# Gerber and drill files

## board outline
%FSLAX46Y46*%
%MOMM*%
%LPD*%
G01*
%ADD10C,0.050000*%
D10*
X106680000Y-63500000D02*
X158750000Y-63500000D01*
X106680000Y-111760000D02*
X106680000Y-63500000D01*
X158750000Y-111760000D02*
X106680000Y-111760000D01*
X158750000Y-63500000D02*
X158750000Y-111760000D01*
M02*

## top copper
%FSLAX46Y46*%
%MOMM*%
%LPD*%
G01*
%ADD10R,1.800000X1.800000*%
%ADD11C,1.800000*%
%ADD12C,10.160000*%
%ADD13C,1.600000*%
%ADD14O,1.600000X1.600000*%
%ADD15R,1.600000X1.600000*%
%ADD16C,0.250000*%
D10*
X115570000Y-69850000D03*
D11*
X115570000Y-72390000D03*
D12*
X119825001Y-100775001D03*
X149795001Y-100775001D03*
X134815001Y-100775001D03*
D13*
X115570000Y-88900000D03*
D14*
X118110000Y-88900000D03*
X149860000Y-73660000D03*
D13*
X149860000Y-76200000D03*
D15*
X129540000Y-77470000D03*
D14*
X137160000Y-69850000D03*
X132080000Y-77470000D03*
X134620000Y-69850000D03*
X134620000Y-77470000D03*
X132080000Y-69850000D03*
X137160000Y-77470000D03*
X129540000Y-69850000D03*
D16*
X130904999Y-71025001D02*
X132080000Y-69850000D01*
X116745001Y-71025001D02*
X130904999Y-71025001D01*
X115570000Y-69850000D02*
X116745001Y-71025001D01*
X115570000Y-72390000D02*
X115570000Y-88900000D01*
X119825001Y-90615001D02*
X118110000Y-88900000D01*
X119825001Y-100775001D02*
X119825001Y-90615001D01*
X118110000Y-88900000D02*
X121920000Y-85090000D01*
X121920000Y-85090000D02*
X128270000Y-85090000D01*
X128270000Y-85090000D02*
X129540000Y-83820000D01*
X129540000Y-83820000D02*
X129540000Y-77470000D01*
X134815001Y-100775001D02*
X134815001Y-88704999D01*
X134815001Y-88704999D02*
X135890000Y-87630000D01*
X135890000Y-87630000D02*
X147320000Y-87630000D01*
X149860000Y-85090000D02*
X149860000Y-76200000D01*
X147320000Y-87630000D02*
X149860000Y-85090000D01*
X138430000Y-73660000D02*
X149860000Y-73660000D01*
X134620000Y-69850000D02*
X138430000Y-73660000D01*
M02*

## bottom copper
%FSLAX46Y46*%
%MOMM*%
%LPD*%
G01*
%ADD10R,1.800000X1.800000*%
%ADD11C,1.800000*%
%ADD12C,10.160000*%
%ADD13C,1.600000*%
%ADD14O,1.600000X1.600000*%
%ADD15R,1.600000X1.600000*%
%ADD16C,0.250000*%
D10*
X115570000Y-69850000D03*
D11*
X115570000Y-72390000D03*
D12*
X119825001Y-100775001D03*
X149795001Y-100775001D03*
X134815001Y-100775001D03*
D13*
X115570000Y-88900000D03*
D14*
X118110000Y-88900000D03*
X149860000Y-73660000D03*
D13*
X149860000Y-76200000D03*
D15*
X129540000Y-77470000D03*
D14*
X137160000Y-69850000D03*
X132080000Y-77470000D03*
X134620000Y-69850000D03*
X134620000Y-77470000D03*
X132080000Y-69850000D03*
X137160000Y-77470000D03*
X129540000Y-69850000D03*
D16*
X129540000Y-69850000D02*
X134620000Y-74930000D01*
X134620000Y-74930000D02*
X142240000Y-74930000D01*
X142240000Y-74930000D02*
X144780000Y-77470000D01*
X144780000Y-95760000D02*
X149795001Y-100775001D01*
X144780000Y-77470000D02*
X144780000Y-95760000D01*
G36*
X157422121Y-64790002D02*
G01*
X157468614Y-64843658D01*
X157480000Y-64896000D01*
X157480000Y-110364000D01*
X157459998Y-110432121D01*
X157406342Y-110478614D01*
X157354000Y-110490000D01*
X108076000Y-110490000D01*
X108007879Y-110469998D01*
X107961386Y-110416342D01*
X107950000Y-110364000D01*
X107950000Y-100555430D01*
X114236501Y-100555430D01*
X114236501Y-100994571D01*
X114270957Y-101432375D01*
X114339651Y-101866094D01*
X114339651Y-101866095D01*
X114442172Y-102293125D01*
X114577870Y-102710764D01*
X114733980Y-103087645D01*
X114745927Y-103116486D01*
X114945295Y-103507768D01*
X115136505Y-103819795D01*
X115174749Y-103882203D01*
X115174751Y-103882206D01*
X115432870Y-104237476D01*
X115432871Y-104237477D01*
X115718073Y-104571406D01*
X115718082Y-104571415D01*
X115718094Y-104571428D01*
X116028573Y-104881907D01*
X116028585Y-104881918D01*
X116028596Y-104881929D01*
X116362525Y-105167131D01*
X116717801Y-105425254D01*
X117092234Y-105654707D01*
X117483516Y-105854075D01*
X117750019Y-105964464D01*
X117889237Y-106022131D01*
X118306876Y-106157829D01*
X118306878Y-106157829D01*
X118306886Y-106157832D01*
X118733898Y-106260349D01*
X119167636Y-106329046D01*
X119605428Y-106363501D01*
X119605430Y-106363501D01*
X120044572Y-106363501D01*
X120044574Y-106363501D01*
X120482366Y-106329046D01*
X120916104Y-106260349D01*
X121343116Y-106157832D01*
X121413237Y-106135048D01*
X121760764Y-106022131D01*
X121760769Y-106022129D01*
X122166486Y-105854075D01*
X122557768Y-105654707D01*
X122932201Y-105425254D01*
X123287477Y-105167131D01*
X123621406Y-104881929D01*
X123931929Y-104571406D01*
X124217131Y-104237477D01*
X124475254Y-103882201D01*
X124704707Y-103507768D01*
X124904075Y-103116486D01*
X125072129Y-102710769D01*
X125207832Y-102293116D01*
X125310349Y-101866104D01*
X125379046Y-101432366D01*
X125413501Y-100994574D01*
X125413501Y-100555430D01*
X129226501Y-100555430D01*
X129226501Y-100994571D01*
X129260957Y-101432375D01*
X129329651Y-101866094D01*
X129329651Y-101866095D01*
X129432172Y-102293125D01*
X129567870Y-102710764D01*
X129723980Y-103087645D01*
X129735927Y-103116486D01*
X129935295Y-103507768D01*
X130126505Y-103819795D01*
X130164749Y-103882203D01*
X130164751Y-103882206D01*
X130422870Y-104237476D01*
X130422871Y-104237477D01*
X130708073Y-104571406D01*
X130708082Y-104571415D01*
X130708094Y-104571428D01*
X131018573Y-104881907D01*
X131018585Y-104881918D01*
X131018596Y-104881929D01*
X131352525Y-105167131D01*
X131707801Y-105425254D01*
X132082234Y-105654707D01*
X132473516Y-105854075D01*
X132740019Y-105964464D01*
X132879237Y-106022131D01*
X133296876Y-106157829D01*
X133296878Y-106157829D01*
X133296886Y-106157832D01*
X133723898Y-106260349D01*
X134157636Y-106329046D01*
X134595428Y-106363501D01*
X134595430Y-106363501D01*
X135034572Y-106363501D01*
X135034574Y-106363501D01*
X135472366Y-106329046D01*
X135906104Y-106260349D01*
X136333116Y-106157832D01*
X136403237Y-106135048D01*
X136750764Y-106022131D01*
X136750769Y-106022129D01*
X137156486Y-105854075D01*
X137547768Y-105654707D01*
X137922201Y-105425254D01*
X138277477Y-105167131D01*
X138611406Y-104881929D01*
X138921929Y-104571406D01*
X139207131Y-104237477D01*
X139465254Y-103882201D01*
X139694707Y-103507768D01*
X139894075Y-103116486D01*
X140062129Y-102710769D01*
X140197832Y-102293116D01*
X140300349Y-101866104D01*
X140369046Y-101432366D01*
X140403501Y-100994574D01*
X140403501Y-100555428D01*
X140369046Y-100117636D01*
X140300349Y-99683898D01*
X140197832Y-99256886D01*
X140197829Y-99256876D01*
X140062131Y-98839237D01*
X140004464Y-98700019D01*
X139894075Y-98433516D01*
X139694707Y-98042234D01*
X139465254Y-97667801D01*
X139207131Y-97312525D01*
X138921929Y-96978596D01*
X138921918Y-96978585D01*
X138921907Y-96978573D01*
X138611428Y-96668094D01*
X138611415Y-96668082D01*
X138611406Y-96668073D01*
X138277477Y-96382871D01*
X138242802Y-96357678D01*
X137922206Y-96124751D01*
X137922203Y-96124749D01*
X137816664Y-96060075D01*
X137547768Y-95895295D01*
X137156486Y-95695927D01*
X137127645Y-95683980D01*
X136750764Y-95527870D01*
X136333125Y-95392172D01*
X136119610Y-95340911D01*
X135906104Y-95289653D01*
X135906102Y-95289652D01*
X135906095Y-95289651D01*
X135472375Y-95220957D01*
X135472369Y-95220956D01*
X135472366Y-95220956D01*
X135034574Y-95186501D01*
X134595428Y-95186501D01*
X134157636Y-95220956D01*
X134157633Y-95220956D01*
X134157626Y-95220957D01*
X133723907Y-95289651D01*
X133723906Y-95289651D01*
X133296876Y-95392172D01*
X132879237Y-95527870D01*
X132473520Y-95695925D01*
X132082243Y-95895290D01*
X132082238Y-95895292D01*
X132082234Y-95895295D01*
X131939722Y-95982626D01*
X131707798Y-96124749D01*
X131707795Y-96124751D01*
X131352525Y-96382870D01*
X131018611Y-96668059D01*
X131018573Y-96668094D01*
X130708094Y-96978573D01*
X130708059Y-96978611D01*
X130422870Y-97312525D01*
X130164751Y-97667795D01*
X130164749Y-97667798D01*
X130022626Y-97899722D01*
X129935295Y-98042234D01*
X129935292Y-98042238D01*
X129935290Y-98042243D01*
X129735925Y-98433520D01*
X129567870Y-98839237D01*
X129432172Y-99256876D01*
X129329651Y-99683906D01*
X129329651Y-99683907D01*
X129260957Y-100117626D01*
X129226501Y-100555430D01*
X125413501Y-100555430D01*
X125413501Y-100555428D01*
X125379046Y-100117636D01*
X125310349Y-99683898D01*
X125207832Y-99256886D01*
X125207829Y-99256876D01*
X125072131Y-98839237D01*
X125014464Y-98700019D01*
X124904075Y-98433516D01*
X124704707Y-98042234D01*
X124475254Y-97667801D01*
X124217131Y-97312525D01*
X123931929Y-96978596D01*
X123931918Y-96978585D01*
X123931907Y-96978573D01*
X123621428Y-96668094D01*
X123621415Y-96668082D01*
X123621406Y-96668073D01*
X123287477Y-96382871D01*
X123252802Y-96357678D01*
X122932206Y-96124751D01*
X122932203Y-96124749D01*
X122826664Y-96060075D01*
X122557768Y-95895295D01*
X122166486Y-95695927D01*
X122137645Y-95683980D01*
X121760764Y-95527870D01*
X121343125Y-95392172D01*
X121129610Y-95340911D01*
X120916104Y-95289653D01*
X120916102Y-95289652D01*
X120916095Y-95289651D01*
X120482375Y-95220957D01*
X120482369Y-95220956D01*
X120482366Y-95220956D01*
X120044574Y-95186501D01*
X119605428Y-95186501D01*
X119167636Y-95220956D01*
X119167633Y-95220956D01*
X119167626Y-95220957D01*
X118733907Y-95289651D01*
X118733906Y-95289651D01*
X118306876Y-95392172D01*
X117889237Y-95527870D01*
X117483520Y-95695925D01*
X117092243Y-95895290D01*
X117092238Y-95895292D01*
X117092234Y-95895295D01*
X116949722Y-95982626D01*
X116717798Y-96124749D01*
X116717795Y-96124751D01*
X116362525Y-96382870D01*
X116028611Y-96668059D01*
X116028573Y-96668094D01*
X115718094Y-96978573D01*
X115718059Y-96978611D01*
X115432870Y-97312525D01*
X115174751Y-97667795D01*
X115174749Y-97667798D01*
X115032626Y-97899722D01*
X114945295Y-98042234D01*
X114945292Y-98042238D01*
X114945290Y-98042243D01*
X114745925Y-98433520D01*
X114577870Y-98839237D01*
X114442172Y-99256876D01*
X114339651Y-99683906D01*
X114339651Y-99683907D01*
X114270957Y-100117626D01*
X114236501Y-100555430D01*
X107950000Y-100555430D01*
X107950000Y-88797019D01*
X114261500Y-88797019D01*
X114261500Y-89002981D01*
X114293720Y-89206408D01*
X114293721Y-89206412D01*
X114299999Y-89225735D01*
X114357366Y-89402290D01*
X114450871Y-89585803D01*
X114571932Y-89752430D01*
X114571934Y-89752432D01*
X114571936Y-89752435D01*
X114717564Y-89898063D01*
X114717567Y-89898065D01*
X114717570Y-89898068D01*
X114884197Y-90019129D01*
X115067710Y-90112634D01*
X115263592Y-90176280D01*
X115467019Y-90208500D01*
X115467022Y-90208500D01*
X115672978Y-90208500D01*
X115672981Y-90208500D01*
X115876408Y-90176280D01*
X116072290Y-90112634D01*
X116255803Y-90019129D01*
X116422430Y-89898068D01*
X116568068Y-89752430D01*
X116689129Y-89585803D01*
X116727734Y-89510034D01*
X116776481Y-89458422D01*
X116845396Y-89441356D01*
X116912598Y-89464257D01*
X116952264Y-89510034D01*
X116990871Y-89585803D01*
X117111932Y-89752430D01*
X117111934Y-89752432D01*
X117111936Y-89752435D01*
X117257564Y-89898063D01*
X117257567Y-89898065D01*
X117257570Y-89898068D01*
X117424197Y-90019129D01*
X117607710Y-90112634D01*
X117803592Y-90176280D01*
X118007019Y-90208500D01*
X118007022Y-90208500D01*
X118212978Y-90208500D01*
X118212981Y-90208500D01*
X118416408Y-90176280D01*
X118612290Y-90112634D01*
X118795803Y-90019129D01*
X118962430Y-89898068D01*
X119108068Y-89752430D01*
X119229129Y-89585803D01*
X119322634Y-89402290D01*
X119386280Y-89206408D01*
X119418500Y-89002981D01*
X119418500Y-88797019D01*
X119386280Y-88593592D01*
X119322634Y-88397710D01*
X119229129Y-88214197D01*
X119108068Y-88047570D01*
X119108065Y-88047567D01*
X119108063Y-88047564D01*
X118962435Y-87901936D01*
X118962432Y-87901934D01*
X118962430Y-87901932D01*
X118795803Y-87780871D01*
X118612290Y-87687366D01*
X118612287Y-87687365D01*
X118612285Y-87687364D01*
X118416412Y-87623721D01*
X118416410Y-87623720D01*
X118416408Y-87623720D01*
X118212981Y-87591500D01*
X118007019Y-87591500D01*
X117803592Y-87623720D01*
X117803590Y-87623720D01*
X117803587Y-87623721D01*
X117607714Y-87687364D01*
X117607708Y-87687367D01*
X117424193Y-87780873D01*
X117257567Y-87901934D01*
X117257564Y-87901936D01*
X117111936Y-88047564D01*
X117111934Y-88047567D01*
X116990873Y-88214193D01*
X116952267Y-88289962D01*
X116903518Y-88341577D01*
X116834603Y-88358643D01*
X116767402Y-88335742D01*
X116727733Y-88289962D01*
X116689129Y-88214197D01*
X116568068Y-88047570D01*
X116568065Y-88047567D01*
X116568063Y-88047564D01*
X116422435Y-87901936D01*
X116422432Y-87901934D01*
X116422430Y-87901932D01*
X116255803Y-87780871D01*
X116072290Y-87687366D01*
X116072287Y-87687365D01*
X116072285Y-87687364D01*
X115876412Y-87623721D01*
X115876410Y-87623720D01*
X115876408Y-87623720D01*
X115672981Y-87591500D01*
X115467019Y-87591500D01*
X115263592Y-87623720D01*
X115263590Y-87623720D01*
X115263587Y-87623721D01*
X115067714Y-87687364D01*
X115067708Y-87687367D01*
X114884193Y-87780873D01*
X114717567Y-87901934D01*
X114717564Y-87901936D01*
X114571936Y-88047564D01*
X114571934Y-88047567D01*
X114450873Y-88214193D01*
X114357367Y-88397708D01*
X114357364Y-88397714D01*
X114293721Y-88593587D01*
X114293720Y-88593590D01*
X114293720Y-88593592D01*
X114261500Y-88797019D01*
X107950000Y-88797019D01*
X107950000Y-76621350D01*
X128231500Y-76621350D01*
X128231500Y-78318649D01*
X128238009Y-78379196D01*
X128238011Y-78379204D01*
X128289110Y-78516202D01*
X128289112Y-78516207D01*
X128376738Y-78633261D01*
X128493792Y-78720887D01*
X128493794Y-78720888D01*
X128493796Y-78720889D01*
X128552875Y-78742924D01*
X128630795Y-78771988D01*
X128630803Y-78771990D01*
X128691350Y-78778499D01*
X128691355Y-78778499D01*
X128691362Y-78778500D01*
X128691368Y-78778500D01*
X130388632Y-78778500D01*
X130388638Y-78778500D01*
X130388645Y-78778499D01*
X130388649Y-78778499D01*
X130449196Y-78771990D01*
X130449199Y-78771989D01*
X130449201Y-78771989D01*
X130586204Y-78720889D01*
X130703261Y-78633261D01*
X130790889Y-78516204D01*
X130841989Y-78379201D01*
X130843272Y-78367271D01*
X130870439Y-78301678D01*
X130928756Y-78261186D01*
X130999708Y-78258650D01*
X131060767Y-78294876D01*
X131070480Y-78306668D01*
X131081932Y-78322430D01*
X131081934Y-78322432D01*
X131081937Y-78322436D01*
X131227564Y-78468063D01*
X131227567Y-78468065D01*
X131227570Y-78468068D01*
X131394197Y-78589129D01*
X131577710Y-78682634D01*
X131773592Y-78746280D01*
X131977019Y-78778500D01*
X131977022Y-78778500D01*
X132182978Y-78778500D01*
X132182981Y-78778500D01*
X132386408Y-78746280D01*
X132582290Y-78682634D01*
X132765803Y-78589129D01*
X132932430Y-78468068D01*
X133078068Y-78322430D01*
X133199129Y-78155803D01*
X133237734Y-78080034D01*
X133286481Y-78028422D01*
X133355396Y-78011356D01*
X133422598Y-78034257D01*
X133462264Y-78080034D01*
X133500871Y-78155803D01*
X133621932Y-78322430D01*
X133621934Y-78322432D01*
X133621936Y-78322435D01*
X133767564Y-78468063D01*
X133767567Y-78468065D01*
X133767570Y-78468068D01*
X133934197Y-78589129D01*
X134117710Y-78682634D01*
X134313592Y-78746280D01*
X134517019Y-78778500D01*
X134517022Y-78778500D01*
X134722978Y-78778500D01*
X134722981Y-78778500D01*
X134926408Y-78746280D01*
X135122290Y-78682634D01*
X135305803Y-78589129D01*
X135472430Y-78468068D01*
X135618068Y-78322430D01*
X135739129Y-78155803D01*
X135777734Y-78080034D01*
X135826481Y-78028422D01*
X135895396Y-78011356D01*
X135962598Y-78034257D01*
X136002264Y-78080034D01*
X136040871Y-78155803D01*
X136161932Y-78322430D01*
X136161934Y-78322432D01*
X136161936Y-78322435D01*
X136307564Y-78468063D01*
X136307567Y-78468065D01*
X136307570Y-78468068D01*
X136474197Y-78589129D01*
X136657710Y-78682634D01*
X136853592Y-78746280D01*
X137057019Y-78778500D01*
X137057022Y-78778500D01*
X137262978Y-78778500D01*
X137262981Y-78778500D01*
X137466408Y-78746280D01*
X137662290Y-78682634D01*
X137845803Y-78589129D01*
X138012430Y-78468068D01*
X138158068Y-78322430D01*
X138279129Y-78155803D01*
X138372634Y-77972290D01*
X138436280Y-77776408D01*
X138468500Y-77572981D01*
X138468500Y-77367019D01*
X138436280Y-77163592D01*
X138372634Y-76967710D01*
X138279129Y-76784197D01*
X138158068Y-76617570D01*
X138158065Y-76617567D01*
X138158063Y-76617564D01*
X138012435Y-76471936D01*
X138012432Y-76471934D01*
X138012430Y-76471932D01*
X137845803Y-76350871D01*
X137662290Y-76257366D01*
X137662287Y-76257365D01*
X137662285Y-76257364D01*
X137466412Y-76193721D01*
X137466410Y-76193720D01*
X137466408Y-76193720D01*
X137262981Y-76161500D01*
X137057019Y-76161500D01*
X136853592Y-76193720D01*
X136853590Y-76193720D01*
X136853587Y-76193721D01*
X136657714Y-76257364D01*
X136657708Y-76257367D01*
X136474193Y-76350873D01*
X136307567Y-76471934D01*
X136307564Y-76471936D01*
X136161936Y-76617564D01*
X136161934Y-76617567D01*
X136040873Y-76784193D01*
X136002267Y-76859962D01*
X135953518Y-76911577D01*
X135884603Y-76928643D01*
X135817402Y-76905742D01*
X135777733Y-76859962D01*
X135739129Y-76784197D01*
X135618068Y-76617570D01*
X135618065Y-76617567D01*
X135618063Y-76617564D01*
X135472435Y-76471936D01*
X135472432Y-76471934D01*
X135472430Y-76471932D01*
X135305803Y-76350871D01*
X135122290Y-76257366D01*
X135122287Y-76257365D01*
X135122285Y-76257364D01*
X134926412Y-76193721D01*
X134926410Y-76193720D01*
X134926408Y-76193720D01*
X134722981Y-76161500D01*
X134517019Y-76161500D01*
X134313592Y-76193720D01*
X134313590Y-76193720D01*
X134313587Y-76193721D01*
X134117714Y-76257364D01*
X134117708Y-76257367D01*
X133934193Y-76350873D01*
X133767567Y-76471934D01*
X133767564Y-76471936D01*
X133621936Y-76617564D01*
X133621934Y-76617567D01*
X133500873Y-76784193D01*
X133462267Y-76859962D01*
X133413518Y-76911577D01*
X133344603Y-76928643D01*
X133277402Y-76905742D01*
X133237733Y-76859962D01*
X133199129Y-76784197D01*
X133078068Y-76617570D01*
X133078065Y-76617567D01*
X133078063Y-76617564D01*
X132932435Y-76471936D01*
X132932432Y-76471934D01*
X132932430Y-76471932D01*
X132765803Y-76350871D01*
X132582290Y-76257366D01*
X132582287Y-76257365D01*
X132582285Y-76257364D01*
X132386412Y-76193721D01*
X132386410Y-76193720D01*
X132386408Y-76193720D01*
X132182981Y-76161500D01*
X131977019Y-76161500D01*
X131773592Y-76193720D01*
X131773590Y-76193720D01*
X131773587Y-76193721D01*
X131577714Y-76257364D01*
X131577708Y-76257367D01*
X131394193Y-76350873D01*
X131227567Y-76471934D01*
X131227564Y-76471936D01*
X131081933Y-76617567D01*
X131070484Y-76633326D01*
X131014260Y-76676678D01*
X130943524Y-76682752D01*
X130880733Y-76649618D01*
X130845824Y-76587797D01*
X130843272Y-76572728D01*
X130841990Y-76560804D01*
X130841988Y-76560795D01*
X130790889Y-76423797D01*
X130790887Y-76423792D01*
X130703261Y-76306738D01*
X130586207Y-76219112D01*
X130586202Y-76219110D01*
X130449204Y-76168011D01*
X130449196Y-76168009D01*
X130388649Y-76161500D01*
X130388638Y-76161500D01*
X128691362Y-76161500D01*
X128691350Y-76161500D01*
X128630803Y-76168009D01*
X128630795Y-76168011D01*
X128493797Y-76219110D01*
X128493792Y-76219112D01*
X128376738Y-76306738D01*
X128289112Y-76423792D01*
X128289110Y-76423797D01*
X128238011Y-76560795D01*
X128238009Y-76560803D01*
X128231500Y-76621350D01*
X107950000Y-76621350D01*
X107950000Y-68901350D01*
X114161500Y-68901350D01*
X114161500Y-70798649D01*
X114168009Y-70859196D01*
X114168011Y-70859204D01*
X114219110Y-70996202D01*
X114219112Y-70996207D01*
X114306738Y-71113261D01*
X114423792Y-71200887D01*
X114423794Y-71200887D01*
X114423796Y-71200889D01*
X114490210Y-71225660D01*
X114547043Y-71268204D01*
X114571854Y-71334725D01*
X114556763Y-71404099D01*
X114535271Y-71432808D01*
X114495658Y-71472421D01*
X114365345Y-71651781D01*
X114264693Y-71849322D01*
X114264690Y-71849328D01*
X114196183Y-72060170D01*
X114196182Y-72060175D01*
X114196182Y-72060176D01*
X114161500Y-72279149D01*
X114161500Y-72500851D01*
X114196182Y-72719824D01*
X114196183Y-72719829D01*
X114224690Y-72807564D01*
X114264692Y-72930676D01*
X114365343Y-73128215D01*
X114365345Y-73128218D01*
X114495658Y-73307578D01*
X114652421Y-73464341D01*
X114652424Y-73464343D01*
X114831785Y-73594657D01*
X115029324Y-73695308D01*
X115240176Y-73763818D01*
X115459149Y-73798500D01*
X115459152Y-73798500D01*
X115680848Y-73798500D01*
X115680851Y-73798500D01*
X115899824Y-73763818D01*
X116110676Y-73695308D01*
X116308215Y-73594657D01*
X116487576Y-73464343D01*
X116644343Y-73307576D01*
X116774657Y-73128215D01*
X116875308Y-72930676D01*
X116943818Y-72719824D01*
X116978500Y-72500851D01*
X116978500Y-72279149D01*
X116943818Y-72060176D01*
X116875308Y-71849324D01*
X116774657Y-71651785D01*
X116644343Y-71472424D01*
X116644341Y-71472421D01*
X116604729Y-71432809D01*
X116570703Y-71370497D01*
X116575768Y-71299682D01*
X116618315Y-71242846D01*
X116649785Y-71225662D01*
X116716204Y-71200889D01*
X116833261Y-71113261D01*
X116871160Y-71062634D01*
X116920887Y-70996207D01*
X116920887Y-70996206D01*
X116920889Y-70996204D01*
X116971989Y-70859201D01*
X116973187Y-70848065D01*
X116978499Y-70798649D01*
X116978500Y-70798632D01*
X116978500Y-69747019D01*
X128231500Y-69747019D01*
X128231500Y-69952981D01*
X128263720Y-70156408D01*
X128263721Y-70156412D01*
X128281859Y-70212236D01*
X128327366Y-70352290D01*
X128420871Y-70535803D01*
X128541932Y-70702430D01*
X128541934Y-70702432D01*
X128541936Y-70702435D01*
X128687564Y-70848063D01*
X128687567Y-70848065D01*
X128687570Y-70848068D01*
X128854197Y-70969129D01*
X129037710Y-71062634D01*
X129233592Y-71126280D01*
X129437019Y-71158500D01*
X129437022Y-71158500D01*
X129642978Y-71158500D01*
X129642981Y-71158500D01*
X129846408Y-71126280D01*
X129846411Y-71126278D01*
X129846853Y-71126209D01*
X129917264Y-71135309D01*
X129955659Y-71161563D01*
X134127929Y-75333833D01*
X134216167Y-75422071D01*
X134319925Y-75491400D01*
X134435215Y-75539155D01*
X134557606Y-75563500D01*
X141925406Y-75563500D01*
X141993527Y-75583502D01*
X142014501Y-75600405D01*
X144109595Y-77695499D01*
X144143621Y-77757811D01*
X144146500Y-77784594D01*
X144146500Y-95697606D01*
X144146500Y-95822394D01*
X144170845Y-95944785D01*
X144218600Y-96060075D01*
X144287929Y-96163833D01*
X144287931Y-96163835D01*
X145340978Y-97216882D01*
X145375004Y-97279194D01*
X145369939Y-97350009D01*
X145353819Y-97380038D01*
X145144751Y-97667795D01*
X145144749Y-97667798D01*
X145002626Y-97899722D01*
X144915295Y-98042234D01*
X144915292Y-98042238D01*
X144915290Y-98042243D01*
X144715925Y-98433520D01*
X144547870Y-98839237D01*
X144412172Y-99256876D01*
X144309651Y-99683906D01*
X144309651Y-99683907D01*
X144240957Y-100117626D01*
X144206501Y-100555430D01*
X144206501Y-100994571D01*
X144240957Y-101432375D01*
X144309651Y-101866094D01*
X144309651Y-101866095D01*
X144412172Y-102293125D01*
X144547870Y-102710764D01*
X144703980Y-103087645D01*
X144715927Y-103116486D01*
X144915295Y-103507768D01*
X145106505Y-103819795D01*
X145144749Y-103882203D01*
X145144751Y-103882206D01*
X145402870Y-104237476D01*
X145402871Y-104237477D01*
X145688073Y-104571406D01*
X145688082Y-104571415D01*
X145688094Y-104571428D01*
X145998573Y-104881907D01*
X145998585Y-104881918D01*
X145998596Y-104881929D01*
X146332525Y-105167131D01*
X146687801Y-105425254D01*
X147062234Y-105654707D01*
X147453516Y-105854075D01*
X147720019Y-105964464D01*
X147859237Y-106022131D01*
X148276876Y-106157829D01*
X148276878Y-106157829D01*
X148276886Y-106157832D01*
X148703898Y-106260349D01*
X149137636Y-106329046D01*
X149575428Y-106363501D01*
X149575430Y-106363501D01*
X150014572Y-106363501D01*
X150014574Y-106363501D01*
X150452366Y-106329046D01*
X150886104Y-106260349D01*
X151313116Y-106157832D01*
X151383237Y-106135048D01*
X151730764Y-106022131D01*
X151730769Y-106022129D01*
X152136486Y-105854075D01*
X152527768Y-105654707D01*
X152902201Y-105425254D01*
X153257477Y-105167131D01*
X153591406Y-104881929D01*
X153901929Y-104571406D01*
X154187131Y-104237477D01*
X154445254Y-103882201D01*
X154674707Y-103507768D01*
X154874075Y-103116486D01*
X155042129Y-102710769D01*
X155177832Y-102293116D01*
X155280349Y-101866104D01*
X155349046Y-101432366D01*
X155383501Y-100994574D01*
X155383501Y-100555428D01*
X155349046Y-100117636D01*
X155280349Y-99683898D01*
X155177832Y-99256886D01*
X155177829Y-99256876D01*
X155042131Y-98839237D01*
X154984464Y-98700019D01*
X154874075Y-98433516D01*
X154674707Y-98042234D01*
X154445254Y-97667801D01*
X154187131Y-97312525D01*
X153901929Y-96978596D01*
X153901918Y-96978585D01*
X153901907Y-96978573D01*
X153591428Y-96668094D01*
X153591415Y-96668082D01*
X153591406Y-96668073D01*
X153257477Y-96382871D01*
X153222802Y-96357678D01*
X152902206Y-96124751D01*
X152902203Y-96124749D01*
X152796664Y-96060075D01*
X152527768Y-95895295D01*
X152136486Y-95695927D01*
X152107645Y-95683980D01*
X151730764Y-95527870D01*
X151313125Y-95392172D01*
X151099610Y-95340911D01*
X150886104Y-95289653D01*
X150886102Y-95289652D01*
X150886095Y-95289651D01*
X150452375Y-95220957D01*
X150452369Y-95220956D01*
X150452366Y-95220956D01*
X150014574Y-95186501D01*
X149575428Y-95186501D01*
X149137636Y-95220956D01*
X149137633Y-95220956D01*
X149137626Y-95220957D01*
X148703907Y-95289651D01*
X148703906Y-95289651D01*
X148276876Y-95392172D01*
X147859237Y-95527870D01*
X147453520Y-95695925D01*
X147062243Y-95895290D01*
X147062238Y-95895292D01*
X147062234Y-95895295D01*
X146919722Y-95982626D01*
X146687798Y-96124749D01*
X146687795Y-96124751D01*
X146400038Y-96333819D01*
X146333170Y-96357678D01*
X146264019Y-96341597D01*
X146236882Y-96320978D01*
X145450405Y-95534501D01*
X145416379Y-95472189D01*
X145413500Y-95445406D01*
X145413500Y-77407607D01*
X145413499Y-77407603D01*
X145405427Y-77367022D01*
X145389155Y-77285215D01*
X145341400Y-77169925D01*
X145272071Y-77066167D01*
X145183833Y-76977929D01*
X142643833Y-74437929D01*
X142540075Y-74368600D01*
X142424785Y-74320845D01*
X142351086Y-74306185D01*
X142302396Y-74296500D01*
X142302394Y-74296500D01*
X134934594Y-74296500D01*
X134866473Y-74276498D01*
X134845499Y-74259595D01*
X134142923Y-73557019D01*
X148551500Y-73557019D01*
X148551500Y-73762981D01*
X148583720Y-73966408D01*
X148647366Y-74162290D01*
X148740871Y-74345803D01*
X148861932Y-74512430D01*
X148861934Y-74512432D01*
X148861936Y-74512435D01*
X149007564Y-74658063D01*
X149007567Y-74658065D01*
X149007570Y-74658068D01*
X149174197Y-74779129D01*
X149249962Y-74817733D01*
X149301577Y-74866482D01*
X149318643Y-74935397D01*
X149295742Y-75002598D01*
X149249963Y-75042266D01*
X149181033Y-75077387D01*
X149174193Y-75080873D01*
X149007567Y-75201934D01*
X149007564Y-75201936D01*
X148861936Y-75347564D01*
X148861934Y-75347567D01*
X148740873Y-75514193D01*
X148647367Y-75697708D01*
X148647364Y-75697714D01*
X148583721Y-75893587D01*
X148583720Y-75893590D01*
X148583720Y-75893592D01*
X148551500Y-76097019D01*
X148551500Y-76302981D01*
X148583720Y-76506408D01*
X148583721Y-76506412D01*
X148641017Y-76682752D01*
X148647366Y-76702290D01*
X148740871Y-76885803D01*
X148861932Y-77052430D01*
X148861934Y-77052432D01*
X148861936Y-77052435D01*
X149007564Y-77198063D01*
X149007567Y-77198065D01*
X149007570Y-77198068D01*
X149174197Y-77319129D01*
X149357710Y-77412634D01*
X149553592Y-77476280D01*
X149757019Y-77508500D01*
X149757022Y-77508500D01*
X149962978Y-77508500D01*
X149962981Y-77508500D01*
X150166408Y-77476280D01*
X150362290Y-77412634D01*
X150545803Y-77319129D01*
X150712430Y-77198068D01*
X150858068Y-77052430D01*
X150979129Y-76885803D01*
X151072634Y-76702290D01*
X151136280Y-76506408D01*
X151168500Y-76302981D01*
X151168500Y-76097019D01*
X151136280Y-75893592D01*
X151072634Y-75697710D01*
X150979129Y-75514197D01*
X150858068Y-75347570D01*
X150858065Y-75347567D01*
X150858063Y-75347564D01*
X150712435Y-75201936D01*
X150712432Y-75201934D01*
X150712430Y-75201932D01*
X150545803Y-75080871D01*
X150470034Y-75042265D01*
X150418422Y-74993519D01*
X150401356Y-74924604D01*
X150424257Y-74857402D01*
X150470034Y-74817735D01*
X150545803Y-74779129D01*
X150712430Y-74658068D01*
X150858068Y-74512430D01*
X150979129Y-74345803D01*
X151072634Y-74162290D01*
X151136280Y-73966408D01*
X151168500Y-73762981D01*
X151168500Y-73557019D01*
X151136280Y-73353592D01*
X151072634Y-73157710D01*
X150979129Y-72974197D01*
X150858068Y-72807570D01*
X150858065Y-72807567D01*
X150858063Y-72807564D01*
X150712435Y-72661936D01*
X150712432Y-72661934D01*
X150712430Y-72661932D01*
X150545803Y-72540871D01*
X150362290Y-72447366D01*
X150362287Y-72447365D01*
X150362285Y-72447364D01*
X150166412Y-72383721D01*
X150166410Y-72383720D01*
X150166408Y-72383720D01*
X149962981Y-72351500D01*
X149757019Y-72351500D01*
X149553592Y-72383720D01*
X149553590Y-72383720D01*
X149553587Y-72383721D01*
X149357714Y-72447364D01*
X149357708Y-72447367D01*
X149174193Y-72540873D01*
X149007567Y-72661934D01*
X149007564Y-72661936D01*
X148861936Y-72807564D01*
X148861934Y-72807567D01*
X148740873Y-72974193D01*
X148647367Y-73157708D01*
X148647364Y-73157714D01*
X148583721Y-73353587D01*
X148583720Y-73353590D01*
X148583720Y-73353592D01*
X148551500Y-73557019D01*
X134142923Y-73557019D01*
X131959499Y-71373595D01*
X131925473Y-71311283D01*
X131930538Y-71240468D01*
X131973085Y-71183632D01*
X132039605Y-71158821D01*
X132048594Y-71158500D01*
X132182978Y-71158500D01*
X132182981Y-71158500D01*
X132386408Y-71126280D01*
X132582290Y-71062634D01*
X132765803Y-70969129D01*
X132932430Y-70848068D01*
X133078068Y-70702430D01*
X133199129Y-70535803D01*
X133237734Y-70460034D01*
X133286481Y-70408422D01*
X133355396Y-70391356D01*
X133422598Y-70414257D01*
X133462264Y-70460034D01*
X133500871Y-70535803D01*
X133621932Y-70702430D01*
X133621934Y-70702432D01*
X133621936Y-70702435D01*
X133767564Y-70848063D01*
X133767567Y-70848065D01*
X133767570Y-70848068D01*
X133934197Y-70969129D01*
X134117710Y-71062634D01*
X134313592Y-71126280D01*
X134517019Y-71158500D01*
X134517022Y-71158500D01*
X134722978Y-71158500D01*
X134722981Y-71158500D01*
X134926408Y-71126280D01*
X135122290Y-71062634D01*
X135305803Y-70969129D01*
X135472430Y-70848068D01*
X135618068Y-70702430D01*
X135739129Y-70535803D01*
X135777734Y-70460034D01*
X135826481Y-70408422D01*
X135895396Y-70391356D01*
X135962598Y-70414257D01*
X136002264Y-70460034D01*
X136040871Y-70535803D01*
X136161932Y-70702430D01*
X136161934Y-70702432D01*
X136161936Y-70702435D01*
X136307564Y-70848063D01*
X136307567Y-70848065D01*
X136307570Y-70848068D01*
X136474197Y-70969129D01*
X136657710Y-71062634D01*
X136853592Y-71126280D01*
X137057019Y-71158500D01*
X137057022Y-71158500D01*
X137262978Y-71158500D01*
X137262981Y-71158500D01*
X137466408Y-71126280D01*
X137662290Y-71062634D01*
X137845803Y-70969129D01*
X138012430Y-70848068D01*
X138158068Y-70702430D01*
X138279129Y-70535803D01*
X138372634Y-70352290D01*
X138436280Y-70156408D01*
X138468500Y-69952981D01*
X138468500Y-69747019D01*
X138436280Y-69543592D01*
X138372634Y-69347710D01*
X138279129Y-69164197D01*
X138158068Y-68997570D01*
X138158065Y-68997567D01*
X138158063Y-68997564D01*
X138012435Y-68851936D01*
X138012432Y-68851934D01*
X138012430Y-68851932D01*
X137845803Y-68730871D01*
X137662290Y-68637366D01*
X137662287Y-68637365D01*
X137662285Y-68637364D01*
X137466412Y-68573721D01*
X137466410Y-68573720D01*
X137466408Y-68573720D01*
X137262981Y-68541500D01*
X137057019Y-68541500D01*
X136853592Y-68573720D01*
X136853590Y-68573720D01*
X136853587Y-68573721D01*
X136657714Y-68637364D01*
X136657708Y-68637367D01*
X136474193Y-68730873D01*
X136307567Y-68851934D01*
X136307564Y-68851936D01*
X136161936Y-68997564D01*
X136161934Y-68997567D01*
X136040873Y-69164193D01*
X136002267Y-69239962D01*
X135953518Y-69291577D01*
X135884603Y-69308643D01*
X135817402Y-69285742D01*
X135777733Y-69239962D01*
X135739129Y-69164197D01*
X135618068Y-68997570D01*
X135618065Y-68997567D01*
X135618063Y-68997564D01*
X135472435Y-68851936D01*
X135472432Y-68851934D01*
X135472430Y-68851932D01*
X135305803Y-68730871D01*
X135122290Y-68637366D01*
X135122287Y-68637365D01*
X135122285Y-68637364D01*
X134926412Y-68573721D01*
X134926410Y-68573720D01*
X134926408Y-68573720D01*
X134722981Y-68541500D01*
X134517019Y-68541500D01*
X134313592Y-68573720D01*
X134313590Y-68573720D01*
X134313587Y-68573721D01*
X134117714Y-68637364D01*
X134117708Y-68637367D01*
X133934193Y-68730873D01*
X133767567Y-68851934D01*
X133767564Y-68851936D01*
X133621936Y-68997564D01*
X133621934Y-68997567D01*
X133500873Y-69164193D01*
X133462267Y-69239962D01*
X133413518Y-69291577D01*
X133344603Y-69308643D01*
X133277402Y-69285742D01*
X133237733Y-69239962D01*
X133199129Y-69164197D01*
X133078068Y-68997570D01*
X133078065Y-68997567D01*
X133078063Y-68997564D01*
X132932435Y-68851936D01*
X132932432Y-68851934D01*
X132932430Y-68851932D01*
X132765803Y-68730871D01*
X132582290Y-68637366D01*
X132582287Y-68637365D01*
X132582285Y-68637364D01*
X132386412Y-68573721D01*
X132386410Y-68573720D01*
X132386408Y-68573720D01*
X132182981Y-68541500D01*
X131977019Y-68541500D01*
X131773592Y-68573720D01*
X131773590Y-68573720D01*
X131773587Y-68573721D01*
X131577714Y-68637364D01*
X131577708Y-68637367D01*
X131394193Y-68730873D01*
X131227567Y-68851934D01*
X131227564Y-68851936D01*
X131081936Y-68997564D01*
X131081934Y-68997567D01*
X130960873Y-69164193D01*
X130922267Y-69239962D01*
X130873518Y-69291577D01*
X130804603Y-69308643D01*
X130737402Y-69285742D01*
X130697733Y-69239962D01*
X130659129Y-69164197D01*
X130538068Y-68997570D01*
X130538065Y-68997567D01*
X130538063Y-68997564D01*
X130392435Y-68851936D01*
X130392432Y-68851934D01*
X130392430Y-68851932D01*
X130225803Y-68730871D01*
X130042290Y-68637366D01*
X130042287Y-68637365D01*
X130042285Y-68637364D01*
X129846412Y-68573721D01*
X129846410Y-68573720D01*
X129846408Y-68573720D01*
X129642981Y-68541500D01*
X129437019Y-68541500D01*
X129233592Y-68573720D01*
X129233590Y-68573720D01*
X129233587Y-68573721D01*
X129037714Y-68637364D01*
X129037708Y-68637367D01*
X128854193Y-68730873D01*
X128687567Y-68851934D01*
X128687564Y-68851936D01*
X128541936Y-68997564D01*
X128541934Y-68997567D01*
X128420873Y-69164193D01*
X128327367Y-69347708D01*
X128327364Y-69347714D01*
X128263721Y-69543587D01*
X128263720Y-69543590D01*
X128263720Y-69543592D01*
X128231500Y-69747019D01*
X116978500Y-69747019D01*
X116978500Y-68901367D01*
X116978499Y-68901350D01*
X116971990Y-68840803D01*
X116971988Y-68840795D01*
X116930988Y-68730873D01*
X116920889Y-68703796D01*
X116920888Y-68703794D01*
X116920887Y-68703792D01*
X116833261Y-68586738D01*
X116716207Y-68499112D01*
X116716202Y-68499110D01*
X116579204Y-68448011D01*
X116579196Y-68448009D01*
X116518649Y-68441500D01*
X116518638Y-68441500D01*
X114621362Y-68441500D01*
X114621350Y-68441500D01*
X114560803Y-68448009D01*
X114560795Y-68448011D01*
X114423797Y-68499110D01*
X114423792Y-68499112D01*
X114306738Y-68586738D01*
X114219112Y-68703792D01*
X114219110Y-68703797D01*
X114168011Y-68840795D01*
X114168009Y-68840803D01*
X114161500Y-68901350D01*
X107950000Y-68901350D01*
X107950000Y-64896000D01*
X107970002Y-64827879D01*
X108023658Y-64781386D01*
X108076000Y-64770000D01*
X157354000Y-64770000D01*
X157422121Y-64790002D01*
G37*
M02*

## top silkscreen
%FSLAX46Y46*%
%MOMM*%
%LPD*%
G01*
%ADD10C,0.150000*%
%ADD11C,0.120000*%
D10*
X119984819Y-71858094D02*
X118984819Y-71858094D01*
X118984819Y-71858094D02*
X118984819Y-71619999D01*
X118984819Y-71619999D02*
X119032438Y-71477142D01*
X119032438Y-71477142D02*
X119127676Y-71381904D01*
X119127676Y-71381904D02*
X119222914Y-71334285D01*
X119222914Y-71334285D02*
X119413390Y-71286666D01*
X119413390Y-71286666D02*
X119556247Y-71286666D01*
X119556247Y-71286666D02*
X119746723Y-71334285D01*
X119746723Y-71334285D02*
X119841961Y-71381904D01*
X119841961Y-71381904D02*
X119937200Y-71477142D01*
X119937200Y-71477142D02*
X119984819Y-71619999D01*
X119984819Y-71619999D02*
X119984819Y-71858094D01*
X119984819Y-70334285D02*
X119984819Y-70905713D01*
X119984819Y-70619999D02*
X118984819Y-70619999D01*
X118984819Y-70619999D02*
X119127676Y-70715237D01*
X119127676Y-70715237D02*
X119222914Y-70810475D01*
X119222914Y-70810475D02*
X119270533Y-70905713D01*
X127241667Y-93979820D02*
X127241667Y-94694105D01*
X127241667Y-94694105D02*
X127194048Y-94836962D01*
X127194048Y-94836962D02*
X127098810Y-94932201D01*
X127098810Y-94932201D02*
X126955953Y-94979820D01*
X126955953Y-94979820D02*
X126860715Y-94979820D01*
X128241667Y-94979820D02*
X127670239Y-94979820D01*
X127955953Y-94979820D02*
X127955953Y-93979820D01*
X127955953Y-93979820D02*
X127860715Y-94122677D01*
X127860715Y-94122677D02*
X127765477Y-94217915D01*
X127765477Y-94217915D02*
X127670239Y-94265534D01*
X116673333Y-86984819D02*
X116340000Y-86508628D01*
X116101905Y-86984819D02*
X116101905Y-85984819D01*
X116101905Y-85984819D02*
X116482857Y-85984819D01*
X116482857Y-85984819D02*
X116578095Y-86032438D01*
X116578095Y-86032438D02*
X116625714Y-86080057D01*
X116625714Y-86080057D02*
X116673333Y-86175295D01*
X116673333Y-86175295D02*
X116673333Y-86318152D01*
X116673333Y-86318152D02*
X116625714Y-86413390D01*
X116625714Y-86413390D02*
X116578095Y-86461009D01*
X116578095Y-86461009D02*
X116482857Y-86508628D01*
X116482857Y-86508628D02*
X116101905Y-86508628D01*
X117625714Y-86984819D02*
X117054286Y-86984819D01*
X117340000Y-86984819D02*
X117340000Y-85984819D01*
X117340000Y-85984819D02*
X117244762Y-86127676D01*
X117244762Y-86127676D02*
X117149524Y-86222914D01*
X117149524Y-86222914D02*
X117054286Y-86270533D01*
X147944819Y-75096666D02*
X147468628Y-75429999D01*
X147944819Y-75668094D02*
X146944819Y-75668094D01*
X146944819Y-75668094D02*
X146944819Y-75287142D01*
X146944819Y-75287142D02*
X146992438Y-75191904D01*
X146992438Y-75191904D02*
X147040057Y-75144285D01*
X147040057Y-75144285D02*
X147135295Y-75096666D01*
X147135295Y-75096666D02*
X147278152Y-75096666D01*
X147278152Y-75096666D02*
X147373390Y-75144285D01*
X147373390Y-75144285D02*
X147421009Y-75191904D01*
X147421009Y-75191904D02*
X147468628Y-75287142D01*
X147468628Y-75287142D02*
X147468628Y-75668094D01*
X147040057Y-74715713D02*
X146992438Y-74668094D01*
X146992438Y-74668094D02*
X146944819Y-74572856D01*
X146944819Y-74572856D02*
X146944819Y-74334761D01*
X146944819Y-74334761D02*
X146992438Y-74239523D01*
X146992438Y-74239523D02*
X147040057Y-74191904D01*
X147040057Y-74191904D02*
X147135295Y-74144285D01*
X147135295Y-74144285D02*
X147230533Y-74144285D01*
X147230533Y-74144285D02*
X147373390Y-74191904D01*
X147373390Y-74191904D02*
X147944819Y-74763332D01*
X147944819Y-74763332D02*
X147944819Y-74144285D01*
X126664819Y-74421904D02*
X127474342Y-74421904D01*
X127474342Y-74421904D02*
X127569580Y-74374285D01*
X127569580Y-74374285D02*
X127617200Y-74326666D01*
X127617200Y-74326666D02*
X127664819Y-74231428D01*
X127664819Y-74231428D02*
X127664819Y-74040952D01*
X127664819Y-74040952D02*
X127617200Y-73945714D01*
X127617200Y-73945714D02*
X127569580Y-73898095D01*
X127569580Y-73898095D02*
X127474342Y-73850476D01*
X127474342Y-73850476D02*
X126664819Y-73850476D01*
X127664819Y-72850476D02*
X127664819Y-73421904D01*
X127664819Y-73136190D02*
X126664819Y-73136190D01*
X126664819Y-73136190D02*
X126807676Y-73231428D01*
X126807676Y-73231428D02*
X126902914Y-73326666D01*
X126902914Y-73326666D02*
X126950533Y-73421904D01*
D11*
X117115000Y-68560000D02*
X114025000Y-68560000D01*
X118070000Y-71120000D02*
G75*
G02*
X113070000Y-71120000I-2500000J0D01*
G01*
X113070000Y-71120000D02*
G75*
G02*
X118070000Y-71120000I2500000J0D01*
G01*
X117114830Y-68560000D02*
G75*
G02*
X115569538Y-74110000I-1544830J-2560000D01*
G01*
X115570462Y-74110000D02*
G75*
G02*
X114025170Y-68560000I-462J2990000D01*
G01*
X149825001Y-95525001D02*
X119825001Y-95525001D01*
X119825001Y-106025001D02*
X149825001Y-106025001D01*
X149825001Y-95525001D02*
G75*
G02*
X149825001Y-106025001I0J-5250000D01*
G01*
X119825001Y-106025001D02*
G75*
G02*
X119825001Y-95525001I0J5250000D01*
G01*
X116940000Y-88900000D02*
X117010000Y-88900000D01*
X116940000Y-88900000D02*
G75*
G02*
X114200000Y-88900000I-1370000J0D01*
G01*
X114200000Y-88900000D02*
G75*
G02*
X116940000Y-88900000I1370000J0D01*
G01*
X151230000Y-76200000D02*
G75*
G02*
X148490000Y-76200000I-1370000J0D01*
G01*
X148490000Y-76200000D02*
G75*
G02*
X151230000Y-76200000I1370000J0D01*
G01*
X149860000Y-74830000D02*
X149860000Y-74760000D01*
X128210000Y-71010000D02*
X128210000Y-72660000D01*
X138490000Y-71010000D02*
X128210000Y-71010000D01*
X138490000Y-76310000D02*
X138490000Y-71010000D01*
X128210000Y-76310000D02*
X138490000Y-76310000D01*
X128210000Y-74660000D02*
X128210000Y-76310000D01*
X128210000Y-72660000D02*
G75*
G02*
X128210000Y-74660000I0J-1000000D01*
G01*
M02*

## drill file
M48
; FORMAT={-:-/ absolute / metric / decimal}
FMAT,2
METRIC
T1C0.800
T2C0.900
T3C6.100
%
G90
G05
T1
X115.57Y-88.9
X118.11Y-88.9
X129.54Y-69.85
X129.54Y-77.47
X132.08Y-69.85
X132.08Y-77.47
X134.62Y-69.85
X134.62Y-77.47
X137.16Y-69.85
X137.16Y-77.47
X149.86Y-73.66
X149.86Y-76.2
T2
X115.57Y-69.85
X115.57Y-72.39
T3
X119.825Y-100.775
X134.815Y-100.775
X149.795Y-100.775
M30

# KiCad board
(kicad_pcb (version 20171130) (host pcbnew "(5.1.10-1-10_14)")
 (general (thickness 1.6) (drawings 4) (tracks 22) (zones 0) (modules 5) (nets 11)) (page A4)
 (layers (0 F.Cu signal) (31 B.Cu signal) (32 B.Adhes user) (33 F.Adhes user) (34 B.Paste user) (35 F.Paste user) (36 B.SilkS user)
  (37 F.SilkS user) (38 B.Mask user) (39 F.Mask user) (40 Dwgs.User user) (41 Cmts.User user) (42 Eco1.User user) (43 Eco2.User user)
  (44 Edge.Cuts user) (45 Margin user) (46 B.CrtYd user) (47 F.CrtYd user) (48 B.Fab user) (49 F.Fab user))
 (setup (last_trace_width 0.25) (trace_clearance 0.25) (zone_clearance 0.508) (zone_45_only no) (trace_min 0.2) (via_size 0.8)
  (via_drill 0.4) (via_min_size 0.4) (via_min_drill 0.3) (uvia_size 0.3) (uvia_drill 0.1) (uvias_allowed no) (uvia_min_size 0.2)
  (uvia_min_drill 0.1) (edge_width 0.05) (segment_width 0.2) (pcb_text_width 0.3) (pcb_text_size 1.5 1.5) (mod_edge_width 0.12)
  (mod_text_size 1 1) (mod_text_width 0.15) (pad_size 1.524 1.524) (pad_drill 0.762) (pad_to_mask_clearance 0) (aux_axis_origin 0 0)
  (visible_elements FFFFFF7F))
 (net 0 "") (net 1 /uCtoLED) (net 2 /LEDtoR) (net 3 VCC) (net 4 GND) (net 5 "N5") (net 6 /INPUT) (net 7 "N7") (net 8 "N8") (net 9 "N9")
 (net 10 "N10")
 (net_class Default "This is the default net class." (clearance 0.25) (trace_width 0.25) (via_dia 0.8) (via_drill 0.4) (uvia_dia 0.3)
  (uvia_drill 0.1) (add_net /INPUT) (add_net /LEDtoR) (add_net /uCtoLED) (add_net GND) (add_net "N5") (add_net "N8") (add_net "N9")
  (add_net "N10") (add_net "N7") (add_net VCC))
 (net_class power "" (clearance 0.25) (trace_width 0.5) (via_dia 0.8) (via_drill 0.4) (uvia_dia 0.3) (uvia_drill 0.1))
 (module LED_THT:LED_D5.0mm (layer F.Cu) (at 115.57 69.85 270)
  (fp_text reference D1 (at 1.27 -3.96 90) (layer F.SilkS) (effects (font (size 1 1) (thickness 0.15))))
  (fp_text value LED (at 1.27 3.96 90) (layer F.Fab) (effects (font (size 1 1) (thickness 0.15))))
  (fp_line (start -1.29 -1.545) (end -1.29 1.545) (layer F.SilkS) (width 0.12))
  (fp_circle (center 1.27 0) (end 3.77 0) (layer F.SilkS) (width 0.12))
  (fp_arc (start 1.27 0) (end -1.29 -1.54483) (angle 148.9) (layer F.SilkS) (width 0.12))
  (fp_arc (start 1.27 0) (end -1.29 1.54483) (angle -148.9) (layer F.SilkS) (width 0.12))
  (pad 1 thru_hole rect (at 0 0 270) (size 1.8 1.8) (drill 0.9) (layers *.Cu *.Mask) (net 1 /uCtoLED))
  (pad 2 thru_hole circle (at 2.54 0 270) (size 1.8 1.8) (drill 0.9) (layers *.Cu *.Mask) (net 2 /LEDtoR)))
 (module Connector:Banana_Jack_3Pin (layer F.Cu) (at 119.825001 100.775001)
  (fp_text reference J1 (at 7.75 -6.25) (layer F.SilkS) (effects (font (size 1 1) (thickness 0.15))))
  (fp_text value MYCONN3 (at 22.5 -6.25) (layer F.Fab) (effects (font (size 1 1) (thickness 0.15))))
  (fp_line (start 30 -5.25) (end 0 -5.25) (layer F.SilkS) (width 0.12))
  (fp_line (start 0 5.25) (end 30 5.25) (layer F.SilkS) (width 0.12))
  (fp_arc (start 30 0) (end 30 -5.25) (angle 180) (layer F.SilkS) (width 0.12))
  (fp_arc (start 0 0) (end 0 5.25) (angle 180) (layer F.SilkS) (width 0.12))
  (pad 1 thru_hole circle (at 0 0) (size 10.16 10.16) (drill 6.1) (layers *.Cu *.Mask) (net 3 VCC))
  (pad 3 thru_hole circle (at 29.97 0) (size 10.16 10.16) (drill 6.1) (layers *.Cu *.Mask) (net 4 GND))
  (pad 2 thru_hole circle (at 14.99 0) (size 10.16 10.16) (drill 6.1) (layers *.Cu *.Mask) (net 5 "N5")))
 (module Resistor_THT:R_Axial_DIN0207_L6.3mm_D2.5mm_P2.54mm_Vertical (layer F.Cu) (at 115.57 88.9)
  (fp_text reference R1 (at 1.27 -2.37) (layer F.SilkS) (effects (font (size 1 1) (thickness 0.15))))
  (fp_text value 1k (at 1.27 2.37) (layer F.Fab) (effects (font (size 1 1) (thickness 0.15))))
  (fp_line (start 1.37 0) (end 1.44 0) (layer F.SilkS) (width 0.12))
  (fp_circle (center 0 0) (end 1.37 0) (layer F.SilkS) (width 0.12))
  (pad 1 thru_hole circle (at 0 0) (size 1.6 1.6) (drill 0.8) (layers *.Cu *.Mask) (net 2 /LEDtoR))
  (pad 2 thru_hole oval (at 2.54 0) (size 1.6 1.6) (drill 0.8) (layers *.Cu *.Mask) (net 3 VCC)))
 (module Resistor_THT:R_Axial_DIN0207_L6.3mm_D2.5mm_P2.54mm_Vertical (layer F.Cu) (at 149.86 76.2 90)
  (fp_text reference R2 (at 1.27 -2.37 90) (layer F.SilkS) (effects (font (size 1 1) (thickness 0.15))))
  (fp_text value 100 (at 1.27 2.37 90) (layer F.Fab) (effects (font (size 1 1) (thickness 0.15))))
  (fp_circle (center 0 0) (end 1.37 0) (layer F.SilkS) (width 0.12))
  (fp_line (start 1.37 0) (end 1.44 0) (layer F.SilkS) (width 0.12))
  (pad 2 thru_hole oval (at 2.54 0 90) (size 1.6 1.6) (drill 0.8) (layers *.Cu *.Mask) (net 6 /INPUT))
  (pad 1 thru_hole circle (at 0 0 90) (size 1.6 1.6) (drill 0.8) (layers *.Cu *.Mask) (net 5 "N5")))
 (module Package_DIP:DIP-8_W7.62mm (layer F.Cu) (at 129.54 77.47 90)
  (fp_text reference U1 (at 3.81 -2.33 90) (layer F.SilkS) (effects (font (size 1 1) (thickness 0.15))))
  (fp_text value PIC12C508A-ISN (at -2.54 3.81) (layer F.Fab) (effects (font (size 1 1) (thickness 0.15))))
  (fp_line (start 6.46 -1.33) (end 4.81 -1.33) (layer F.SilkS) (width 0.12))
  (fp_line (start 6.46 8.95) (end 6.46 -1.33) (layer F.SilkS) (width 0.12))
  (fp_line (start 1.16 8.95) (end 6.46 8.95) (layer F.SilkS) (width 0.12))
  (fp_line (start 1.16 -1.33) (end 1.16 8.95) (layer F.SilkS) (width 0.12))
  (fp_line (start 2.81 -1.33) (end 1.16 -1.33) (layer F.SilkS) (width 0.12))
  (fp_arc (start 3.81 -1.33) (end 2.81 -1.33) (angle -180) (layer F.SilkS) (width 0.12))
  (pad 1 thru_hole rect (at 0 0 90) (size 1.6 1.6) (drill 0.8) (layers *.Cu *.Mask) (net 3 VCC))
  (pad 5 thru_hole oval (at 7.62 7.62 90) (size 1.6 1.6) (drill 0.8) (layers *.Cu *.Mask) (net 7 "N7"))
  (pad 2 thru_hole oval (at 0 2.54 90) (size 1.6 1.6) (drill 0.8) (layers *.Cu *.Mask) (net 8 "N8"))
  (pad 6 thru_hole oval (at 7.62 5.08 90) (size 1.6 1.6) (drill 0.8) (layers *.Cu *.Mask) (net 6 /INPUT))
  (pad 3 thru_hole oval (at 0 5.08 90) (size 1.6 1.6) (drill 0.8) (layers *.Cu *.Mask) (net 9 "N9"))
  (pad 7 thru_hole oval (at 7.62 2.54 90) (size 1.6 1.6) (drill 0.8) (layers *.Cu *.Mask) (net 1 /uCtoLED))
  (pad 4 thru_hole oval (at 0 7.62 90) (size 1.6 1.6) (drill 0.8) (layers *.Cu *.Mask) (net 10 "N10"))
  (pad 8 thru_hole oval (at 7.62 0 90) (size 1.6 1.6) (drill 0.8) (layers *.Cu *.Mask) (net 4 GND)))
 (gr_line (start 106.68 63.5) (end 158.75 63.5) (layer Edge.Cuts) (width 0.05))
 (gr_line (start 106.68 111.76) (end 106.68 63.5) (layer Edge.Cuts) (width 0.05))
 (gr_line (start 158.75 111.76) (end 106.68 111.76) (layer Edge.Cuts) (width 0.05))
 (gr_line (start 158.75 63.5) (end 158.75 111.76) (layer Edge.Cuts) (width 0.05))
 (segment (start 130.904999 71.025001) (end 132.08 69.85) (width 0.25) (layer F.Cu) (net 1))
 (segment (start 116.745001 71.025001) (end 130.904999 71.025001) (width 0.25) (layer F.Cu) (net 1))
 (segment (start 115.57 69.85) (end 116.745001 71.025001) (width 0.25) (layer F.Cu) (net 1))
 (segment (start 115.57 72.39) (end 115.57 88.9) (width 0.25) (layer F.Cu) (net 2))
 (segment (start 119.825001 90.615001) (end 118.11 88.9) (width 0.25) (layer F.Cu) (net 3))
 (segment (start 119.825001 100.775001) (end 119.825001 90.615001) (width 0.25) (layer F.Cu) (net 3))
 (segment (start 118.11 88.9) (end 121.92 85.09) (width 0.25) (layer F.Cu) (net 3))
 (segment (start 121.92 85.09) (end 128.27 85.09) (width 0.25) (layer F.Cu) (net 3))
 (segment (start 128.27 85.09) (end 129.54 83.82) (width 0.25) (layer F.Cu) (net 3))
 (segment (start 129.54 83.82) (end 129.54 77.47) (width 0.25) (layer F.Cu) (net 3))
 (segment (start 129.54 69.85) (end 134.62 74.93) (width 0.25) (layer B.Cu) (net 4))
 (segment (start 134.62 74.93) (end 142.24 74.93) (width 0.25) (layer B.Cu) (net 4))
 (segment (start 142.24 74.93) (end 144.78 77.47) (width 0.25) (layer B.Cu) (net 4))
 (segment (start 144.78 95.76) (end 149.795001 100.775001) (width 0.25) (layer B.Cu) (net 4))
 (segment (start 144.78 77.47) (end 144.78 95.76) (width 0.25) (layer B.Cu) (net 4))
 (segment (start 134.815001 100.775001) (end 134.815001 88.704999) (width 0.25) (layer F.Cu) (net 5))
 (segment (start 134.815001 88.704999) (end 135.89 87.63) (width 0.25) (layer F.Cu) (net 5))
 (segment (start 135.89 87.63) (end 147.32 87.63) (width 0.25) (layer F.Cu) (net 5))
 (segment (start 149.86 85.09) (end 149.86 76.2) (width 0.25) (layer F.Cu) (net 5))
 (segment (start 147.32 87.63) (end 149.86 85.09) (width 0.25) (layer F.Cu) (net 5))
 (segment (start 138.43 73.66) (end 149.86 73.66) (width 0.25) (layer F.Cu) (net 6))
 (segment (start 134.62 69.85) (end 138.43 73.66) (width 0.25) (layer F.Cu) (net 6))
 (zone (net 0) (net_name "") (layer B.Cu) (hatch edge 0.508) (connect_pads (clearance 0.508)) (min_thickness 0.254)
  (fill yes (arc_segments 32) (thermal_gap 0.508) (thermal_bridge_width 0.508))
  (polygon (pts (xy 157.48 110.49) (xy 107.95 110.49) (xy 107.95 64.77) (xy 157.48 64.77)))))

